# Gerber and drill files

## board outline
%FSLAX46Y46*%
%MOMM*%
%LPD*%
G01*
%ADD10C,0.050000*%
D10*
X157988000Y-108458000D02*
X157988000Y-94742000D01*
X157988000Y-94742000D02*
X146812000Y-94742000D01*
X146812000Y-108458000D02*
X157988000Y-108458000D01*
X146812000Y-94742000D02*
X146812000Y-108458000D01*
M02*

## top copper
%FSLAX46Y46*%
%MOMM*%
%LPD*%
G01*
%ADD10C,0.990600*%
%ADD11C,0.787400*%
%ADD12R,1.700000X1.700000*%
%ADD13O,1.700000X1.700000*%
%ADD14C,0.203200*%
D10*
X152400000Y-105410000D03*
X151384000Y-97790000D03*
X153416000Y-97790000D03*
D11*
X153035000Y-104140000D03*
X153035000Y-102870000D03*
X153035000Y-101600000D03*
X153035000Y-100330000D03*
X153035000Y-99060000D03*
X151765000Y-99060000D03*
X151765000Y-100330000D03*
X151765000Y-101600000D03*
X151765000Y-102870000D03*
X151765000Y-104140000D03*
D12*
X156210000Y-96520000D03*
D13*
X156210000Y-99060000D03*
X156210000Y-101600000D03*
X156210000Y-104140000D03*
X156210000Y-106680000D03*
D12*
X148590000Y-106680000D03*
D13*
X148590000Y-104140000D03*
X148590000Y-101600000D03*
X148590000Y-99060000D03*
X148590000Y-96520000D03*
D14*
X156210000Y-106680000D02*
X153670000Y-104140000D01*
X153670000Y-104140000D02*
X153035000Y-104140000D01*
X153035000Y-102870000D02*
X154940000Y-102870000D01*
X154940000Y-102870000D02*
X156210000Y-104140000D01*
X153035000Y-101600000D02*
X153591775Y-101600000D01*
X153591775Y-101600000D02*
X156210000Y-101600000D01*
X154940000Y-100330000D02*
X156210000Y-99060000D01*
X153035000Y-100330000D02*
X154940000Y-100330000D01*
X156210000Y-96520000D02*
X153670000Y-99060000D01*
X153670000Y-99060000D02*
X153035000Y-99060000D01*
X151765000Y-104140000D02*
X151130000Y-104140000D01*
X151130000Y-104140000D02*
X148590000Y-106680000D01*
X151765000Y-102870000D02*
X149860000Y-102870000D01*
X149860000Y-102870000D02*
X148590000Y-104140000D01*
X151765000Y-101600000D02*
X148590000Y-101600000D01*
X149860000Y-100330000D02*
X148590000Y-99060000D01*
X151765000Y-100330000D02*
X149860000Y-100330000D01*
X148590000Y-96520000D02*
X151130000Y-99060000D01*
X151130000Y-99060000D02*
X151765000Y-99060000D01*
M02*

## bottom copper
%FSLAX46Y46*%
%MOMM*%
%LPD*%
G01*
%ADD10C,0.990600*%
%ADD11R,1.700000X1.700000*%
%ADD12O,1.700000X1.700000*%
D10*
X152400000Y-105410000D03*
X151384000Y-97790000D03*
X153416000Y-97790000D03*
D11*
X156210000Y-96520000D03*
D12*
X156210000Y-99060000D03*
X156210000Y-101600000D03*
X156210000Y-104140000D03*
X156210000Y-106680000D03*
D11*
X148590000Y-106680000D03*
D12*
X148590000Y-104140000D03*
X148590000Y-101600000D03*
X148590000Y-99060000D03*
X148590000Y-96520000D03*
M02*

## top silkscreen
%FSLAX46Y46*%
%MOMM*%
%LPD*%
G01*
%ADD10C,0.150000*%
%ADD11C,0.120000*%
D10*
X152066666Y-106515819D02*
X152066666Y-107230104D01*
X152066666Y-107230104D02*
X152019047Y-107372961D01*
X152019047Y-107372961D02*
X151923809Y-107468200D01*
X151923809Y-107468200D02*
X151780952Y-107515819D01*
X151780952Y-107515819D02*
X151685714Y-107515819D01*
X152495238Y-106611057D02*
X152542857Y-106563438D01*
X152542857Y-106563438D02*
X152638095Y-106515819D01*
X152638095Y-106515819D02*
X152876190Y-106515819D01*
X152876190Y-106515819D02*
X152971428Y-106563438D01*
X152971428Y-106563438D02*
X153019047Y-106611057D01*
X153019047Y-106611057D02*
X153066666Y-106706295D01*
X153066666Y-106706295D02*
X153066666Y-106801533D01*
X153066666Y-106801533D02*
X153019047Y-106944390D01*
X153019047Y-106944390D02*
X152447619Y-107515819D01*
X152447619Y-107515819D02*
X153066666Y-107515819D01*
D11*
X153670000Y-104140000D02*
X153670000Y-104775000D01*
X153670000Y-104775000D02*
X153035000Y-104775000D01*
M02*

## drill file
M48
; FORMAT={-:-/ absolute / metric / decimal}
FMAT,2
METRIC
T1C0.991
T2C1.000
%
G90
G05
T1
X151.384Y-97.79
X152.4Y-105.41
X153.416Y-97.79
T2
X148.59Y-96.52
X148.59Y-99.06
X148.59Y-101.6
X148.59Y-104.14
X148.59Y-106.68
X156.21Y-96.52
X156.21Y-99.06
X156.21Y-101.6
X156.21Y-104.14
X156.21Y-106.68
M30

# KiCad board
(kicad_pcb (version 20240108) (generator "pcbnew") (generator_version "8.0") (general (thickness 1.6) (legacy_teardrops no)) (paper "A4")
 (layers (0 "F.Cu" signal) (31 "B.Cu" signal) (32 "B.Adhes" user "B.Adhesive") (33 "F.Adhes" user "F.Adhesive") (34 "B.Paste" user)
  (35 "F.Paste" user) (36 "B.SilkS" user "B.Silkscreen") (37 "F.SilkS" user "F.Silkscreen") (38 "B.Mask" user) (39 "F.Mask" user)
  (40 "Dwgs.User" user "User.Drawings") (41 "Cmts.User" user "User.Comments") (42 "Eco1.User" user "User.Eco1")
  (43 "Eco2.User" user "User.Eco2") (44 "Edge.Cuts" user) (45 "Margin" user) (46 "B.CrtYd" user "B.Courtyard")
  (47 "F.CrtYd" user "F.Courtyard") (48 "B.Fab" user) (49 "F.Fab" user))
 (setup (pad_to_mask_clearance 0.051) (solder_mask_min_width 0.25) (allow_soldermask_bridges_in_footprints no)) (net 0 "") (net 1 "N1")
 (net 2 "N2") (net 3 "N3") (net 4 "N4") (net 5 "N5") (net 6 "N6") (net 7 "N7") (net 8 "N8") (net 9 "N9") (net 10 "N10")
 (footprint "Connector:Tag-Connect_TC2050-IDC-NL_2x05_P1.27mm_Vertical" (layer "F.Cu") (at 152.4 101.6 90)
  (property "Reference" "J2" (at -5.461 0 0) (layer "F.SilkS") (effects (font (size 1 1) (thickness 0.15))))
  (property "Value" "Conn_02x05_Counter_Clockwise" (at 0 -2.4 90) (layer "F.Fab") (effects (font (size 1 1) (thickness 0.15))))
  (fp_line (start -2.54 1.27) (end -3.175 1.27) (stroke (width 0.12) (type solid)) (layer "F.SilkS"))
  (fp_line (start -3.175 1.27) (end -3.175 0.635) (stroke (width 0.12) (type solid)) (layer "F.SilkS"))
  (pad "" thru_hole circle (at -3.81 0 90) (size 0.9906 0.9906) (drill 0.9906) (layers "*.Cu" "*.Mask") (remove_unused_layers no))
  (pad "" thru_hole circle (at 3.81 -1.016 90) (size 0.9906 0.9906) (drill 0.9906) (layers "*.Cu" "*.Mask") (remove_unused_layers no))
  (pad "" thru_hole circle (at 3.81 1.016 90) (size 0.9906 0.9906) (drill 0.9906) (layers "*.Cu" "*.Mask") (remove_unused_layers no))
  (pad "1" connect circle (at -2.54 0.635 90) (size 0.7874 0.7874) (layers "F.Cu" "F.Mask") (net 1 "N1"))
  (pad "2" connect circle (at -1.27 0.635 90) (size 0.7874 0.7874) (layers "F.Cu" "F.Mask") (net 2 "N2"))
  (pad "3" connect circle (at 0 0.635 90) (size 0.7874 0.7874) (layers "F.Cu" "F.Mask") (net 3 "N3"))
  (pad "4" connect circle (at 1.27 0.635 90) (size 0.7874 0.7874) (layers "F.Cu" "F.Mask") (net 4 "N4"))
  (pad "5" connect circle (at 2.54 0.635 90) (size 0.7874 0.7874) (layers "F.Cu" "F.Mask") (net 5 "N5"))
  (pad "6" connect circle (at 2.54 -0.635 90) (size 0.7874 0.7874) (layers "F.Cu" "F.Mask") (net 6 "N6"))
  (pad "7" connect circle (at 1.27 -0.635 90) (size 0.7874 0.7874) (layers "F.Cu" "F.Mask") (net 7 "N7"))
  (pad "8" connect circle (at 0 -0.635 90) (size 0.7874 0.7874) (layers "F.Cu" "F.Mask") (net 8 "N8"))
  (pad "9" connect circle (at -1.27 -0.635 90) (size 0.7874 0.7874) (layers "F.Cu" "F.Mask") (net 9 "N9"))
  (pad "10" connect circle (at -2.54 -0.635 90) (size 0.7874 0.7874) (layers "F.Cu" "F.Mask") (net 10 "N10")))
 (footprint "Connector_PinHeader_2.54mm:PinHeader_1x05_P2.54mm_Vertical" (layer "B.Cu") (at 156.21 96.52 180)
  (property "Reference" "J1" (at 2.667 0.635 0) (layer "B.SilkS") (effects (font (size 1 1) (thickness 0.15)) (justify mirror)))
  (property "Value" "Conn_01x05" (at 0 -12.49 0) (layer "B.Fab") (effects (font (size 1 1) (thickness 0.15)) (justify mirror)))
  (pad "1" thru_hole rect (at 0 0 180) (size 1.7 1.7) (drill 1) (layers "*.Cu" "*.Mask") (remove_unused_layers no) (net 5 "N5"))
  (pad "2" thru_hole oval (at 0 -2.54 180) (size 1.7 1.7) (drill 1) (layers "*.Cu" "*.Mask") (remove_unused_layers no) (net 4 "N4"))
  (pad "3" thru_hole oval (at 0 -5.08 180) (size 1.7 1.7) (drill 1) (layers "*.Cu" "*.Mask") (remove_unused_layers no) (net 3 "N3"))
  (pad "4" thru_hole oval (at 0 -7.62 180) (size 1.7 1.7) (drill 1) (layers "*.Cu" "*.Mask") (remove_unused_layers no) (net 2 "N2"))
  (pad "5" thru_hole oval (at 0 -10.16 180) (size 1.7 1.7) (drill 1) (layers "*.Cu" "*.Mask") (remove_unused_layers no) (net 1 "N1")))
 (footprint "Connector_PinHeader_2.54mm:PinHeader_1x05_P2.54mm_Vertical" (layer "B.Cu") (at 148.59 106.68)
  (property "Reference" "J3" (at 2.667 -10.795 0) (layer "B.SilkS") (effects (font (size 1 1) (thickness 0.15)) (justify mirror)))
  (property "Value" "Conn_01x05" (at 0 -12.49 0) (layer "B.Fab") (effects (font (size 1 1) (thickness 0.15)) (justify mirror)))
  (pad "1" thru_hole rect (at 0 0) (size 1.7 1.7) (drill 1) (layers "*.Cu" "*.Mask") (remove_unused_layers no) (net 10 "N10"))
  (pad "2" thru_hole oval (at 0 -2.54) (size 1.7 1.7) (drill 1) (layers "*.Cu" "*.Mask") (remove_unused_layers no) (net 9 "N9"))
  (pad "3" thru_hole oval (at 0 -5.08) (size 1.7 1.7) (drill 1) (layers "*.Cu" "*.Mask") (remove_unused_layers no) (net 8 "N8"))
  (pad "4" thru_hole oval (at 0 -7.62) (size 1.7 1.7) (drill 1) (layers "*.Cu" "*.Mask") (remove_unused_layers no) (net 7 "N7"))
  (pad "5" thru_hole oval (at 0 -10.16) (size 1.7 1.7) (drill 1) (layers "*.Cu" "*.Mask") (remove_unused_layers no) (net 6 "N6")))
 (gr_line (start 157.988 108.458) (end 157.988 94.742) (stroke (width 0.05) (type solid)) (layer "Edge.Cuts"))
 (gr_line (start 157.988 94.742) (end 146.812 94.742) (stroke (width 0.05) (type solid)) (layer "Edge.Cuts"))
 (gr_line (start 146.812 108.458) (end 157.988 108.458) (stroke (width 0.05) (type solid)) (layer "Edge.Cuts"))
 (gr_line (start 146.812 94.742) (end 146.812 108.458) (stroke (width 0.05) (type solid)) (layer "Edge.Cuts"))
 (segment (start 156.21 106.68) (end 153.67 104.14) (width 0.2032) (layer "F.Cu") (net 1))
 (segment (start 153.67 104.14) (end 153.035 104.14) (width 0.2032) (layer "F.Cu") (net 1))
 (segment (start 153.035 102.87) (end 154.94 102.87) (width 0.2032) (layer "F.Cu") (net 2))
 (segment (start 154.94 102.87) (end 156.21 104.14) (width 0.2032) (layer "F.Cu") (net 2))
 (segment (start 153.035 101.6) (end 153.591775 101.6) (width 0.2032) (layer "F.Cu") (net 3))
 (segment (start 153.591775 101.6) (end 156.21 101.6) (width 0.2032) (layer "F.Cu") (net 3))
 (segment (start 154.94 100.33) (end 156.21 99.06) (width 0.2032) (layer "F.Cu") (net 4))
 (segment (start 153.035 100.33) (end 154.94 100.33) (width 0.2032) (layer "F.Cu") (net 4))
 (segment (start 156.21 96.52) (end 153.67 99.06) (width 0.2032) (layer "F.Cu") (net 5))
 (segment (start 153.67 99.06) (end 153.035 99.06) (width 0.2032) (layer "F.Cu") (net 5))
 (segment (start 151.765 104.14) (end 151.13 104.14) (width 0.2032) (layer "F.Cu") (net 10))
 (segment (start 151.13 104.14) (end 148.59 106.68) (width 0.2032) (layer "F.Cu") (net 10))
 (segment (start 151.765 102.87) (end 149.86 102.87) (width 0.2032) (layer "F.Cu") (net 9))
 (segment (start 149.86 102.87) (end 148.59 104.14) (width 0.2032) (layer "F.Cu") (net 9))
 (segment (start 151.765 101.6) (end 148.59 101.6) (width 0.2032) (layer "F.Cu") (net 8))
 (segment (start 149.86 100.33) (end 148.59 99.06) (width 0.2032) (layer "F.Cu") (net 7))
 (segment (start 151.765 100.33) (end 149.86 100.33) (width 0.2032) (layer "F.Cu") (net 7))
 (segment (start 148.59 96.52) (end 151.13 99.06) (width 0.2032) (layer "F.Cu") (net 6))
 (segment (start 151.13 99.06) (end 151.765 99.06) (width 0.2032) (layer "F.Cu") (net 6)))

